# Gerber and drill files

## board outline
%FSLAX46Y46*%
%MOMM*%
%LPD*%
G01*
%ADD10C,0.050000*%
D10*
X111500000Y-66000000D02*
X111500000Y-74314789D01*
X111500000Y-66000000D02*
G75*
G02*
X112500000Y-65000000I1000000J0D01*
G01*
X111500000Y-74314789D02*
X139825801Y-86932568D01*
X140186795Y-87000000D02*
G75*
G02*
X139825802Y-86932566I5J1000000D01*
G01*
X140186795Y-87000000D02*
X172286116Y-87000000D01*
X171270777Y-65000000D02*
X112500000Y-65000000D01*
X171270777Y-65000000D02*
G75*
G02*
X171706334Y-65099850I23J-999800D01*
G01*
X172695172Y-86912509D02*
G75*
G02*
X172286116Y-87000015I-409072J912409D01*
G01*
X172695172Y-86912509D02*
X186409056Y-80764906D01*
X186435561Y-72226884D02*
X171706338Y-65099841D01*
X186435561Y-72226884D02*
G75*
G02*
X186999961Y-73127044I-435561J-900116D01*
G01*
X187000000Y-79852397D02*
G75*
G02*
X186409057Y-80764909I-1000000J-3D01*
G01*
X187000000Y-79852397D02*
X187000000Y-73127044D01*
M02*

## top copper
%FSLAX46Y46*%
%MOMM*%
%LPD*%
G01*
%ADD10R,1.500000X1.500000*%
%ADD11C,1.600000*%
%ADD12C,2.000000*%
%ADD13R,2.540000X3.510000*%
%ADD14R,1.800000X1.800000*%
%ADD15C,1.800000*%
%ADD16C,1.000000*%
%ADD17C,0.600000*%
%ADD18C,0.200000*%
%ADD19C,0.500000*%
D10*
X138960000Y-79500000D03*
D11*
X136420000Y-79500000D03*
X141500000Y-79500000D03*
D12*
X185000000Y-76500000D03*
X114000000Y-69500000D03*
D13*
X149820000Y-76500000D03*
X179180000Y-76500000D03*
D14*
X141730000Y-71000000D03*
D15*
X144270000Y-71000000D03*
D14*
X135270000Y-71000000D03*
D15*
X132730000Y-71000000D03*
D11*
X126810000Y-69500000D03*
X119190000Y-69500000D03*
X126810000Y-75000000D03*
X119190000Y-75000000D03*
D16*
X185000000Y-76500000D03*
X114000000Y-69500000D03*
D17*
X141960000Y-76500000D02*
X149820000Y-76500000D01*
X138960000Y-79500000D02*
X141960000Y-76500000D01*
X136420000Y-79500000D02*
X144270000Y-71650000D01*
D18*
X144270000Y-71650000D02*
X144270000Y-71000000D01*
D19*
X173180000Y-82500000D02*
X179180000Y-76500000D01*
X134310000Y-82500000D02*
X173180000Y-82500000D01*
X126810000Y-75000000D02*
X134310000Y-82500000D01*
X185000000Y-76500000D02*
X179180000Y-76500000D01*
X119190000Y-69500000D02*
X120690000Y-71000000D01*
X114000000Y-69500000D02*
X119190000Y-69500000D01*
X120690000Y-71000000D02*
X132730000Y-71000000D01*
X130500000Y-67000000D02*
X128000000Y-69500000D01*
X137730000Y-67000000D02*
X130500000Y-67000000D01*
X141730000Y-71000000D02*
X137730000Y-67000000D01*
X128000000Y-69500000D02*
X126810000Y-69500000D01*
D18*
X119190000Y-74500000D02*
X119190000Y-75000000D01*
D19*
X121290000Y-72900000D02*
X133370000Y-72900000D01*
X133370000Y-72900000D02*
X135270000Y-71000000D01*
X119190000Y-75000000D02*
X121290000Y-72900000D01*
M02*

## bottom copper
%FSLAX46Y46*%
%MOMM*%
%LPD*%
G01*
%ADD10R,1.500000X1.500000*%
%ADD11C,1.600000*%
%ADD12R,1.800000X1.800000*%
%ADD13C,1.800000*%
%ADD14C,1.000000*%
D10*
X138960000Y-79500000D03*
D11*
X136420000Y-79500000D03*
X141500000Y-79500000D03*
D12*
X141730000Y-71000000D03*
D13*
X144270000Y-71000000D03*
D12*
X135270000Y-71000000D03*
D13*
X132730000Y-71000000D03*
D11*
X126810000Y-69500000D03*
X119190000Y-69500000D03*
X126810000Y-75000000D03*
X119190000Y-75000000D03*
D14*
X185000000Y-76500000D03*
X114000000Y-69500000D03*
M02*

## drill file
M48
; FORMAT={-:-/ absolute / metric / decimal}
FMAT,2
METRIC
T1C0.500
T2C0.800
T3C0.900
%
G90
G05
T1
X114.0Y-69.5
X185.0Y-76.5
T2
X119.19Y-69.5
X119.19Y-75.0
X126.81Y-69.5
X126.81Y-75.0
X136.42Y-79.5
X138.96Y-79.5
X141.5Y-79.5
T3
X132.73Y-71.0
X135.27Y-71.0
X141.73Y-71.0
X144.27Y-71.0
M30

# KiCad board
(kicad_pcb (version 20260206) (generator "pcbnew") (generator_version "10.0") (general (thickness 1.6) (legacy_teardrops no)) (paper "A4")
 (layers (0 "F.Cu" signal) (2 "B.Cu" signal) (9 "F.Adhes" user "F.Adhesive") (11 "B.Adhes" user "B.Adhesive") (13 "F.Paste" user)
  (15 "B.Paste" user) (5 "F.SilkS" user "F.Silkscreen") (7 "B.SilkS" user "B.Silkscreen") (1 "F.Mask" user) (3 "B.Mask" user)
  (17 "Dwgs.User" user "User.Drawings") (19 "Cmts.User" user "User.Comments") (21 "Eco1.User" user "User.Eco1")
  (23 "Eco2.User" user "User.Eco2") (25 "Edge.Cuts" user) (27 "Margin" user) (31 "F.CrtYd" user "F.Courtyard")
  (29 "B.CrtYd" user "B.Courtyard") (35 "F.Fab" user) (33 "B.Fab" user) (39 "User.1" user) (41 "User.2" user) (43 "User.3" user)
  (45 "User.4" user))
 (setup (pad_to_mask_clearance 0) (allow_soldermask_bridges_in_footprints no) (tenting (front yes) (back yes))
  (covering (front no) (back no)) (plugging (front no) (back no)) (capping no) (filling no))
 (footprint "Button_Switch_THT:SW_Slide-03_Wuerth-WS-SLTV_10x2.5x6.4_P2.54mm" (layer "F.Cu") (at 138.96 79.5)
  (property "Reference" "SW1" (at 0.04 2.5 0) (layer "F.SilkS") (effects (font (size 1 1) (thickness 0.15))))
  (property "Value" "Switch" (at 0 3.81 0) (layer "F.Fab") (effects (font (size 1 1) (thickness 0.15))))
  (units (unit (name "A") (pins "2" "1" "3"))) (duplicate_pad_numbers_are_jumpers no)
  (pad "1" thru_hole rect (at 0 0) (size 1.5 1.5) (drill 0.8) (layers "*.Cu" "*.Mask") (remove_unused_layers no) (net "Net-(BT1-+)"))
  (pad "2" thru_hole circle (at -2.54 0) (size 1.6 1.6) (drill 0.8) (layers "*.Cu" "*.Mask") (remove_unused_layers no) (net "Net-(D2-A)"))
  (pad "3" thru_hole circle (at 2.54 0) (size 1.6 1.6) (drill 0.8) (layers "*.Cu" "*.Mask") (remove_unused_layers no)
   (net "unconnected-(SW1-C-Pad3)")))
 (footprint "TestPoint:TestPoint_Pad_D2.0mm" (layer "F.Cu") (at 185 76.5)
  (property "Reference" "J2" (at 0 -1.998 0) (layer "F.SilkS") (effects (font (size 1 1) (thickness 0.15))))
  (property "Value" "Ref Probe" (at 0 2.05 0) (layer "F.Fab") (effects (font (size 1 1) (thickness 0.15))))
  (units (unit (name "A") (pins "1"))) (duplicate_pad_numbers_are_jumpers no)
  (pad "1" smd circle (at 0 0) (size 2 2) (layers "F.Cu" "F.Mask") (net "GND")))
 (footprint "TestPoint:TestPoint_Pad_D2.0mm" (layer "F.Cu") (at 114 69.5)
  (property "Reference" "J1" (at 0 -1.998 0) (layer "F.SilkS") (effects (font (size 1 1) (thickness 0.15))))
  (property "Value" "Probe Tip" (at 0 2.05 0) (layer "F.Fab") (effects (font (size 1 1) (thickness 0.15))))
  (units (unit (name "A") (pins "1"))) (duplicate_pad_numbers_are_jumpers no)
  (pad "1" smd circle (at 0 0) (size 2 2) (layers "F.Cu" "F.Mask") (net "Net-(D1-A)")))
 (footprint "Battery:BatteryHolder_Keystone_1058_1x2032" (layer "F.Cu") (at 164.5 76.5)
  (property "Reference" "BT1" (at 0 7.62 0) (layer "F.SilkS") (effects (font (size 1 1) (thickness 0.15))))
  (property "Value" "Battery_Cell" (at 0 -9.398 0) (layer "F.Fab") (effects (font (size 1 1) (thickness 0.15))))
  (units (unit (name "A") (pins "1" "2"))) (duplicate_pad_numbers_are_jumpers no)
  (pad "1" smd rect (at -14.68 0) (size 2.54 3.51) (layers "F.Cu" "F.Mask" "F.Paste") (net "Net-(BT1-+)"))
  (pad "2" smd rect (at 14.68 0) (size 2.54 3.51) (layers "F.Cu" "F.Mask" "F.Paste") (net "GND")))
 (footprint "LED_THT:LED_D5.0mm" (layer "F.Cu") (at 141.73 71)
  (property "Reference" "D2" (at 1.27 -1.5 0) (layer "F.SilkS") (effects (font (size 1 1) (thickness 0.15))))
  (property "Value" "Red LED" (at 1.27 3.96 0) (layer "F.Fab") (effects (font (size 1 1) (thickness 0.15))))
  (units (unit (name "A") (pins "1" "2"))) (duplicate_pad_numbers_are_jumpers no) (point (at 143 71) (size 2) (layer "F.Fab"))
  (pad "1" thru_hole rect (at 0 0) (size 1.8 1.8) (drill 0.9) (layers "*.Cu" "*.Mask") (remove_unused_layers no) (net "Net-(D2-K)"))
  (pad "2" thru_hole circle (at 2.54 0) (size 1.8 1.8) (drill 0.9) (layers "*.Cu" "*.Mask") (remove_unused_layers no) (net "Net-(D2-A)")))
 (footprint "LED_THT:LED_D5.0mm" (layer "F.Cu") (at 135.27 71 180)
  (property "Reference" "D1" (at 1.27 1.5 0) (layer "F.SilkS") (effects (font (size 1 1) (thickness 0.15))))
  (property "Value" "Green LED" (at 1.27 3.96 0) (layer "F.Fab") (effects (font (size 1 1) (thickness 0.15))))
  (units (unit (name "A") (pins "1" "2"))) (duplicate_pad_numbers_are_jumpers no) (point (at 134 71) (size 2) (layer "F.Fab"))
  (pad "1" thru_hole rect (at 0 0 180) (size 1.8 1.8) (drill 0.9) (layers "*.Cu" "*.Mask") (remove_unused_layers no) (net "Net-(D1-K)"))
  (pad "2" thru_hole circle (at 2.54 0 180) (size 1.8 1.8) (drill 0.9) (layers "*.Cu" "*.Mask") (remove_unused_layers no) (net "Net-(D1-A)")))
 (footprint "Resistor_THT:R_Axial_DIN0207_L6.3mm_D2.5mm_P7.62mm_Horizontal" (layer "F.Cu") (at 126.81 69.5 180)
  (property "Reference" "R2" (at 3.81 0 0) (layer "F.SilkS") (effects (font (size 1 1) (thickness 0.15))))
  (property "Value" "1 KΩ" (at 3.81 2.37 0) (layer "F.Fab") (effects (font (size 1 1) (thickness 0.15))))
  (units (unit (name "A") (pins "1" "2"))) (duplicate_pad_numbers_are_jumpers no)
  (pad "1" thru_hole circle (at 0 0 180) (size 1.6 1.6) (drill 0.8) (layers "*.Cu" "*.Mask") (remove_unused_layers no) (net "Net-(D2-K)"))
  (pad "2" thru_hole circle (at 7.62 0 180) (size 1.6 1.6) (drill 0.8) (layers "*.Cu" "*.Mask") (remove_unused_layers no) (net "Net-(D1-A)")))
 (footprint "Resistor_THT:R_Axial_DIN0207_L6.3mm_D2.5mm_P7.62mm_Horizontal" (layer "F.Cu") (at 126.81 75 180)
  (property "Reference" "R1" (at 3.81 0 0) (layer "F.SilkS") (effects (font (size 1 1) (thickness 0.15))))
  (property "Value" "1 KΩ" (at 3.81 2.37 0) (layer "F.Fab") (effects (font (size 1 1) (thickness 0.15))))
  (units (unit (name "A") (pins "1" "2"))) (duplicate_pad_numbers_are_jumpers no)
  (pad "1" thru_hole circle (at 0 0 180) (size 1.6 1.6) (drill 0.8) (layers "*.Cu" "*.Mask") (remove_unused_layers no) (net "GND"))
  (pad "2" thru_hole circle (at 7.62 0 180) (size 1.6 1.6) (drill 0.8) (layers "*.Cu" "*.Mask") (remove_unused_layers no) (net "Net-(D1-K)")))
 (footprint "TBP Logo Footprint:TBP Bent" (layer "F.Cu") (at 150.5 68.5)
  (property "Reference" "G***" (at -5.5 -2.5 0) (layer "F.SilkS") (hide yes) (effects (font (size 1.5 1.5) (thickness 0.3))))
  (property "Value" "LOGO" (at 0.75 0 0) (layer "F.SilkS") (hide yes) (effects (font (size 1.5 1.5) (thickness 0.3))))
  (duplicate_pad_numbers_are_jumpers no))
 (gr_line (start 111.5 66) (end 111.5 74.314789) (stroke (width 0.05) (type default)) (layer "Edge.Cuts"))
 (gr_arc (start 111.5 66) (mid 111.792893 65.292893) (end 112.5 65) (stroke (width 0.05) (type solid)) (layer "Edge.Cuts"))
 (gr_line (start 111.5 74.314789) (end 139.825801 86.932568) (stroke (width 0.05) (type solid)) (layer "Edge.Cuts"))
 (gr_arc (start 140.186795 87) (mid 140.003176 86.982997) (end 139.825801 86.932568) (stroke (width 0.05) (type default))
  (layer "Edge.Cuts"))
 (gr_line (start 140.186795 87) (end 172.286116 87) (stroke (width 0.05) (type default)) (layer "Edge.Cuts"))
 (gr_line (start 171.270777 65) (end 112.5 65) (stroke (width 0.05) (type solid)) (layer "Edge.Cuts"))
 (gr_arc (start 171.270777 65) (mid 171.494207 65.025275) (end 171.706338 65.099841) (stroke (width 0.05) (type default))
  (layer "Edge.Cuts"))
 (gr_arc (start 172.695172 86.912509) (mid 172.49527 86.977886) (end 172.286116 87) (stroke (width 0.05) (type default)) (layer "Edge.Cuts"))
 (gr_line (start 172.695172 86.912509) (end 186.409056 80.764906) (stroke (width 0.05) (type default)) (layer "Edge.Cuts"))
 (gr_line (start 186.435561 72.226884) (end 171.706338 65.099841) (stroke (width 0.05) (type default)) (layer "Edge.Cuts"))
 (gr_arc (start 186.435561 72.226884) (mid 186.84722 72.5958) (end 187 73.127044) (stroke (width 0.05) (type default)) (layer "Edge.Cuts"))
 (gr_arc (start 187 79.852397) (mid 186.839363 80.395972) (end 186.409056 80.764906) (stroke (width 0.05) (type default))
  (layer "Edge.Cuts"))
 (gr_line (start 187 79.852397) (end 187 73.127044) (stroke (width 0.05) (type default)) (layer "Edge.Cuts"))
 (segment (start 141.96 76.5) (end 149.82 76.5) (width 0.6) (layer "F.Cu") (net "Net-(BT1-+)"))
 (segment (start 138.96 79.5) (end 141.96 76.5) (width 0.6) (layer "F.Cu") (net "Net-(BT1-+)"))
 (segment (start 136.42 79.5) (end 144.27 71.65) (width 0.6) (layer "F.Cu") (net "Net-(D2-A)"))
 (segment (start 144.27 71.65) (end 144.27 71) (width 0.2) (layer "F.Cu") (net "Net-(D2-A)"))
 (segment (start 173.18 82.5) (end 179.18 76.5) (width 0.5) (layer "F.Cu") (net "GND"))
 (segment (start 134.31 82.5) (end 173.18 82.5) (width 0.5) (layer "F.Cu") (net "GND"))
 (segment (start 126.81 75) (end 134.31 82.5) (width 0.5) (layer "F.Cu") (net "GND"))
 (segment (start 185 76.5) (end 179.18 76.5) (width 0.5) (layer "F.Cu") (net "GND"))
 (via (at 185 76.5) (size 1) (drill 0.5) (layers "F.Cu" "B.Cu") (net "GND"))
 (segment (start 119.19 69.5) (end 120.69 71) (width 0.5) (layer "F.Cu") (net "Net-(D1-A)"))
 (segment (start 114 69.5) (end 119.19 69.5) (width 0.5) (layer "F.Cu") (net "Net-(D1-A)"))
 (segment (start 120.69 71) (end 132.73 71) (width 0.5) (layer "F.Cu") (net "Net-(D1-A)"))
 (via (at 114 69.5) (size 1) (drill 0.5) (layers "F.Cu" "B.Cu") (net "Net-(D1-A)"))
 (segment (start 130.5 67) (end 128 69.5) (width 0.5) (layer "F.Cu") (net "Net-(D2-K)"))
 (segment (start 137.73 67) (end 130.5 67) (width 0.5) (layer "F.Cu") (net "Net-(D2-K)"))
 (segment (start 141.73 71) (end 137.73 67) (width 0.5) (layer "F.Cu") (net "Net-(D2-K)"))
 (segment (start 128 69.5) (end 126.81 69.5) (width 0.5) (layer "F.Cu") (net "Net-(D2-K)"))
 (segment (start 119.19 74.5) (end 119.19 75) (width 0.2) (layer "F.Cu") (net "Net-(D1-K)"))
 (segment (start 121.29 72.9) (end 133.37 72.9) (width 0.5) (layer "F.Cu") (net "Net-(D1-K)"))
 (segment (start 133.37 72.9) (end 135.27 71) (width 0.5) (layer "F.Cu") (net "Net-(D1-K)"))
 (segment (start 119.19 75) (end 121.29 72.9) (width 0.5) (layer "F.Cu") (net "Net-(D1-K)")))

